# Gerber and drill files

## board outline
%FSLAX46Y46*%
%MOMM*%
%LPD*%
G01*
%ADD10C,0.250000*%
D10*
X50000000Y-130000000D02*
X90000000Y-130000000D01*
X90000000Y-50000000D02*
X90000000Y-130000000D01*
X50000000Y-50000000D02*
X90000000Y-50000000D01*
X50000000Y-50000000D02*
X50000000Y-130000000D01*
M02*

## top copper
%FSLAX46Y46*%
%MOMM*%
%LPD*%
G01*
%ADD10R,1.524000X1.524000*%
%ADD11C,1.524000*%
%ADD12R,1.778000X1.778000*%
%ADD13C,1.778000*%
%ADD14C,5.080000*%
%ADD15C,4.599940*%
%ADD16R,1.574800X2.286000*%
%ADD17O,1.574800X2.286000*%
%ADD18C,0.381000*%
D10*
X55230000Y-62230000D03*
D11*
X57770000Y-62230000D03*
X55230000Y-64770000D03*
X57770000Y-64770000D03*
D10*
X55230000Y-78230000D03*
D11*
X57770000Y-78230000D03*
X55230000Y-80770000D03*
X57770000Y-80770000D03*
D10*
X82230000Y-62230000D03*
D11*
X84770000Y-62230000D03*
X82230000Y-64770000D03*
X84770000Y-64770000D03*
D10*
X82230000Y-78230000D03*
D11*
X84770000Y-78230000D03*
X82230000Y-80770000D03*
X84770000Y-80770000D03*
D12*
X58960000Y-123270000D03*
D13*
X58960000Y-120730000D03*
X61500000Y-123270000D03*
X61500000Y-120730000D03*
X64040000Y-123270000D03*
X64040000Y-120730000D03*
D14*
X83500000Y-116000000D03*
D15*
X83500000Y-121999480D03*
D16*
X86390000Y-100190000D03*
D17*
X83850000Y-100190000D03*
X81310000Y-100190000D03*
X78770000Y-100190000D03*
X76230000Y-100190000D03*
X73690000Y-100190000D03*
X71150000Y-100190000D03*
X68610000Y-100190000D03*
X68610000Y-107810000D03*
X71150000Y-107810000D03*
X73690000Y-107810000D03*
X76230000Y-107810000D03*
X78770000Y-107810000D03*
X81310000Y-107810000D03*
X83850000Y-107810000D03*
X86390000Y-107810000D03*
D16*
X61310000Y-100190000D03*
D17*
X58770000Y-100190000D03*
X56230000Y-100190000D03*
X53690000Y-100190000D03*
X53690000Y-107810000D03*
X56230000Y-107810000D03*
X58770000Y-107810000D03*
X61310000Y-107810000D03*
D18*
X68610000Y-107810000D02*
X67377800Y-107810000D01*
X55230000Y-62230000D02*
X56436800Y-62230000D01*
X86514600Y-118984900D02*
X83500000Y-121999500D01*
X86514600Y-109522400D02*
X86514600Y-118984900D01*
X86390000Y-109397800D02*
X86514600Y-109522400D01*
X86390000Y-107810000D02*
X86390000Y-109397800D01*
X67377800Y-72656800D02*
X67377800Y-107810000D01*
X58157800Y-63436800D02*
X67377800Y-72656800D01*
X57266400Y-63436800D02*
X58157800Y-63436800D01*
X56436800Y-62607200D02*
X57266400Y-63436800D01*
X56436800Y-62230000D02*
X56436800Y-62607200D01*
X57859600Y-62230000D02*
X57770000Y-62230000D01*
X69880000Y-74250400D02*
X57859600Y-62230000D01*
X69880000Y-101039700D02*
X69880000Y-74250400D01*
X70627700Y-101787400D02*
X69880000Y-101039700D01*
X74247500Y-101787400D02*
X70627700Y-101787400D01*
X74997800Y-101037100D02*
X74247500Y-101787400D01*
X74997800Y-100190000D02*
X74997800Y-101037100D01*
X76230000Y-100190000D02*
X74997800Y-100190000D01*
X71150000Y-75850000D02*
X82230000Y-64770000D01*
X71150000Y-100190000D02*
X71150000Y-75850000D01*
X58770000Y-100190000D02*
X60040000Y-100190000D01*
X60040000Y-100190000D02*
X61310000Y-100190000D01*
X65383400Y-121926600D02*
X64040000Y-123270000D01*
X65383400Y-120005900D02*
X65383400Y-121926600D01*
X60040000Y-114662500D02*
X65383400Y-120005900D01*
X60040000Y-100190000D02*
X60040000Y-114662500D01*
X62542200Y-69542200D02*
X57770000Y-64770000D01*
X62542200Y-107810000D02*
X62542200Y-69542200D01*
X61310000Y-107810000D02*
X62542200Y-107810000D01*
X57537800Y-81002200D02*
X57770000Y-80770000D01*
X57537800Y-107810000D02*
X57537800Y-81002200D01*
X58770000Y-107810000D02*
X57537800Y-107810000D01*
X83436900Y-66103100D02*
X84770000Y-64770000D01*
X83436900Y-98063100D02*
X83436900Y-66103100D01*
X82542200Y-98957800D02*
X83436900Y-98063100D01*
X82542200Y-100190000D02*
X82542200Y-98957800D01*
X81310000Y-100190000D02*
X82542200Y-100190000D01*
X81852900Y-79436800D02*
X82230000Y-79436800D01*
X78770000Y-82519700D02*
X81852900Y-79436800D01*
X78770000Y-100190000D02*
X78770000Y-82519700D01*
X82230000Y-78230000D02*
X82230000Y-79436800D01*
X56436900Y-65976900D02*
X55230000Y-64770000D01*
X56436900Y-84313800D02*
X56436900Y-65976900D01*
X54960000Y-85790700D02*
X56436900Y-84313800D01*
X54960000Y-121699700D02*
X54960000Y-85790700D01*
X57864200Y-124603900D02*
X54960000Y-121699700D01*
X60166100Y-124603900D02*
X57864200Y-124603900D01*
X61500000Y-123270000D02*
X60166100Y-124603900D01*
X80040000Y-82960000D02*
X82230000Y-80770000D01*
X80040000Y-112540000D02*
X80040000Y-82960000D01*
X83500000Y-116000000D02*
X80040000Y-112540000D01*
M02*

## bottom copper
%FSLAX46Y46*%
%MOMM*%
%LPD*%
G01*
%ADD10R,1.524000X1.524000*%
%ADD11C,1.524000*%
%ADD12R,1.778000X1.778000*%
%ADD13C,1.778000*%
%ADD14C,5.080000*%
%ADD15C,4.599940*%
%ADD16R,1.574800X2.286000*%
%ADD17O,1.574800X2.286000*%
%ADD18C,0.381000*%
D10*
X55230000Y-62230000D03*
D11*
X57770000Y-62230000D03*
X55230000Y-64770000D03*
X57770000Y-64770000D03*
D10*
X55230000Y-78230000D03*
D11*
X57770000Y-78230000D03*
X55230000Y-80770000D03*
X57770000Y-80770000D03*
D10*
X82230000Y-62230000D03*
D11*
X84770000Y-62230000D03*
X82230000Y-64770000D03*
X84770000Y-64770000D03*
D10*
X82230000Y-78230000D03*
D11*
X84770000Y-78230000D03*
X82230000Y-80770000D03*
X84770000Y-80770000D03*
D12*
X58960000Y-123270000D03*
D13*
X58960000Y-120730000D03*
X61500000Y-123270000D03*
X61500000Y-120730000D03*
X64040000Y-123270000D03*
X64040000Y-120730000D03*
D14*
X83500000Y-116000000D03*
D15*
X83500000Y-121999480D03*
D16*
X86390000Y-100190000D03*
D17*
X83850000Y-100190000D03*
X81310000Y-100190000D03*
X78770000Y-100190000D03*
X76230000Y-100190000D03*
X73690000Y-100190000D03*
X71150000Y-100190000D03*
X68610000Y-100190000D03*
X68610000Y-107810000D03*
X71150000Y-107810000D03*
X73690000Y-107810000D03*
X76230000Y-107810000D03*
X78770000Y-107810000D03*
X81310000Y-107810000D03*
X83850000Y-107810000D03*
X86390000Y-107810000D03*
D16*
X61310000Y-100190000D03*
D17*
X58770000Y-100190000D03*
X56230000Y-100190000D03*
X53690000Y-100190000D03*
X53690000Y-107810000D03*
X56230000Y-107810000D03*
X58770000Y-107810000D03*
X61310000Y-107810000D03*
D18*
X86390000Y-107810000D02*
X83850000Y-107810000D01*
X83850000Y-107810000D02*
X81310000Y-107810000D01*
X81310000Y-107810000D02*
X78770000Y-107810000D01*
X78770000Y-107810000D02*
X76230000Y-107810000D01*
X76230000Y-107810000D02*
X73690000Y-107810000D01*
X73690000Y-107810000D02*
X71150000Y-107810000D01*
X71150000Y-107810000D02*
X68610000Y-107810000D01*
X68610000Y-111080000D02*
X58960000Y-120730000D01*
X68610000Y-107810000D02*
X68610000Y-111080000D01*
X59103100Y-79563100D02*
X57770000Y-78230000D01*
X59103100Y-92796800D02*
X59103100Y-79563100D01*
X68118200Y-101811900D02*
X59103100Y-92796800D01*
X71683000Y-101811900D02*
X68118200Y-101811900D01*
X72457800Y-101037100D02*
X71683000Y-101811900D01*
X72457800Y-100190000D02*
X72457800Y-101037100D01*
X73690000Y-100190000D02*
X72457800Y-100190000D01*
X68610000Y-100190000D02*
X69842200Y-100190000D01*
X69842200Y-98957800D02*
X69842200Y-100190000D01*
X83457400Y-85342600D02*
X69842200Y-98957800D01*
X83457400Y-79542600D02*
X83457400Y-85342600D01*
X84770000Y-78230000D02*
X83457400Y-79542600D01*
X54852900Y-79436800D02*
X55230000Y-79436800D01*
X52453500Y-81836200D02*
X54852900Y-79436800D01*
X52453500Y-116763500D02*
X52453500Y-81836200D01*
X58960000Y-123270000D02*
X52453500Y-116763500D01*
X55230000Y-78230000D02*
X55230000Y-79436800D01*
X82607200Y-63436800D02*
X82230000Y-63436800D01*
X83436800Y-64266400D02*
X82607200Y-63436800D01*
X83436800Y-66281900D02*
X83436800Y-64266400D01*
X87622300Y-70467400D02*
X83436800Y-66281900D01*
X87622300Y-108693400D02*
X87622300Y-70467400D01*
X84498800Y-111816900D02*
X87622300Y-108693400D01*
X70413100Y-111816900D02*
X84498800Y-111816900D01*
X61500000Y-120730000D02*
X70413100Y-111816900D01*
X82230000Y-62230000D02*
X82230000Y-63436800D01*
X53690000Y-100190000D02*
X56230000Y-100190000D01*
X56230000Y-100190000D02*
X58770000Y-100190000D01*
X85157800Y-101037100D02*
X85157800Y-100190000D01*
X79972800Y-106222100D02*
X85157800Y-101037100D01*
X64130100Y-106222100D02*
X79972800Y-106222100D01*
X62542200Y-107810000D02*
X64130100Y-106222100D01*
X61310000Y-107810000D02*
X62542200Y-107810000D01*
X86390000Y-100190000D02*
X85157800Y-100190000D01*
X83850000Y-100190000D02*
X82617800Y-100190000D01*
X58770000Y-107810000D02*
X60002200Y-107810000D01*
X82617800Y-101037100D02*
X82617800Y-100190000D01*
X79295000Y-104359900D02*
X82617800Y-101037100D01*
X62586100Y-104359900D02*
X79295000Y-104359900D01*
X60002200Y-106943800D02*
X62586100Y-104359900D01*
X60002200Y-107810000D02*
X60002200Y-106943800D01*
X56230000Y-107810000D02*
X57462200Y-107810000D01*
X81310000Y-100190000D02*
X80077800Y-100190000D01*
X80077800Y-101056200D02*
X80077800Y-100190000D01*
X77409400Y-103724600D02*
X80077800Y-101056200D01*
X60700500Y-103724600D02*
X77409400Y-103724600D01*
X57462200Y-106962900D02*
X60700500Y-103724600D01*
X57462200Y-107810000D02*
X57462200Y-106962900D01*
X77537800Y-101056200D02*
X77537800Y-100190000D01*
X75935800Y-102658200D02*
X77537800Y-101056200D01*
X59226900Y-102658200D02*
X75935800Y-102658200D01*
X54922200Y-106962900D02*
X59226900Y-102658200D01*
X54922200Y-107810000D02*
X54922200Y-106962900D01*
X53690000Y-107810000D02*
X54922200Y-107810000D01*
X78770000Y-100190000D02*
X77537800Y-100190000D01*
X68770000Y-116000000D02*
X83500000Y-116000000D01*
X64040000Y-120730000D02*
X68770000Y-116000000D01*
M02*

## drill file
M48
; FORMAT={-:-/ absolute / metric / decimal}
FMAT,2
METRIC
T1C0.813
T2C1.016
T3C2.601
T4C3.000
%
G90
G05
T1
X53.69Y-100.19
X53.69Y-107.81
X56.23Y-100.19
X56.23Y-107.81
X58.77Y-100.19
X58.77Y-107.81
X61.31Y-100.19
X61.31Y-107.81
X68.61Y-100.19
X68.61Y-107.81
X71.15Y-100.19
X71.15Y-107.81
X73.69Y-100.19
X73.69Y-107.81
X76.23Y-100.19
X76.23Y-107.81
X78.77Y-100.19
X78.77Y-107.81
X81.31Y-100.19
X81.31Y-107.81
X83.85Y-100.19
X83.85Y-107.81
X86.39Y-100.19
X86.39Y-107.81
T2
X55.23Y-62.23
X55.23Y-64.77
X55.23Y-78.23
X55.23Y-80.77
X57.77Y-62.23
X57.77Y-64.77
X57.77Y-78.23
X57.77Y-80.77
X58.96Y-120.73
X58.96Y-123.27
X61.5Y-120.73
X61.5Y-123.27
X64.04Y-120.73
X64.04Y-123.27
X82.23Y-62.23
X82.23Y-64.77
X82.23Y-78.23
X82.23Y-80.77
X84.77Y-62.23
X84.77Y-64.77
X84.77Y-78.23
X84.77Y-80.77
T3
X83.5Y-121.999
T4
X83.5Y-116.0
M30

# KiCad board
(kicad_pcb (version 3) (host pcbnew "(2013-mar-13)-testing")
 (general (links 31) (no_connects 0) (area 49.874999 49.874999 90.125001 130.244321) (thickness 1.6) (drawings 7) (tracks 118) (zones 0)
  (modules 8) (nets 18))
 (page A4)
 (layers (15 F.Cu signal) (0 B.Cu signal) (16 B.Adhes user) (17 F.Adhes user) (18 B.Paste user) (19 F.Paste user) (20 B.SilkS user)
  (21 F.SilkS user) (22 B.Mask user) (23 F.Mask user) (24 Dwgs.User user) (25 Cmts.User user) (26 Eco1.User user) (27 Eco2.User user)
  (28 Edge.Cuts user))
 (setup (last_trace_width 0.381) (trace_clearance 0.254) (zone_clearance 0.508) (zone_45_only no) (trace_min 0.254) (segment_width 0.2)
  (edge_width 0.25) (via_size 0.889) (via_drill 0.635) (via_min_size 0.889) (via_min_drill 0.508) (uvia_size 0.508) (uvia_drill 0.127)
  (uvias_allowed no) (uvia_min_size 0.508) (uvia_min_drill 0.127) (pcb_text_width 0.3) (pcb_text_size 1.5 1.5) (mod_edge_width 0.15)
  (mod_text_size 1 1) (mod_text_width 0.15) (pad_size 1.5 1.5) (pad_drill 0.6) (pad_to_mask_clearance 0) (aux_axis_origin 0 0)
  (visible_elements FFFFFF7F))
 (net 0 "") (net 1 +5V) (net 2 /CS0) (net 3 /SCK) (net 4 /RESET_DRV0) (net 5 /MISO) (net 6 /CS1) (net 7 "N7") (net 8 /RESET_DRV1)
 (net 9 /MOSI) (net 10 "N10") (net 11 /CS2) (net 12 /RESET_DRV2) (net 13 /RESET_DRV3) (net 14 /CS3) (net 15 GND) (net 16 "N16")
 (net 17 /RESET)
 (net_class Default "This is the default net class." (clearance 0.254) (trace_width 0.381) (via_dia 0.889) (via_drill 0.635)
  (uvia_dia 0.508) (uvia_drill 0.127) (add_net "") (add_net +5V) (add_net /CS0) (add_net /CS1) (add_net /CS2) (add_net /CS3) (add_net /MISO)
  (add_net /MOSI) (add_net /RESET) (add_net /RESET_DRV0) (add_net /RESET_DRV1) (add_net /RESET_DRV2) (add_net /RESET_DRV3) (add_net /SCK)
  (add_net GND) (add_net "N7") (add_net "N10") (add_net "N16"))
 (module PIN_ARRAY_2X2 (layer F.Cu) (at 56.5 63.5 270)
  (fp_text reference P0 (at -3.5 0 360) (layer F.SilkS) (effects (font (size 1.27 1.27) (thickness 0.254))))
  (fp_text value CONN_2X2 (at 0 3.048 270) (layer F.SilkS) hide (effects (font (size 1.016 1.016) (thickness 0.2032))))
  (pad 1 thru_hole rect (at -1.27 1.27 270) (size 1.524 1.524) (drill 1.016) (layers *.Cu *.Mask F.SilkS) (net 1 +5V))
  (pad 2 thru_hole circle (at -1.27 -1.27 270) (size 1.524 1.524) (drill 1.016) (layers *.Cu *.Mask F.SilkS) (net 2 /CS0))
  (pad 3 thru_hole circle (at 1.27 1.27 270) (size 1.524 1.524) (drill 1.016) (layers *.Cu *.Mask F.SilkS) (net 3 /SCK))
  (pad 4 thru_hole circle (at 1.27 -1.27 270) (size 1.524 1.524) (drill 1.016) (layers *.Cu *.Mask F.SilkS) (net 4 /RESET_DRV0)))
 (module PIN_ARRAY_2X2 (layer F.Cu) (at 56.5 79.5 270)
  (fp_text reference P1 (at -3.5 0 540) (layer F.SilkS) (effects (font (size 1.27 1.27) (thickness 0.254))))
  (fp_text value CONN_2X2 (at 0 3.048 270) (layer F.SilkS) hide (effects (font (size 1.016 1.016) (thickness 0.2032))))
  (pad 1 thru_hole rect (at -1.27 1.27 270) (size 1.524 1.524) (drill 1.016) (layers *.Cu *.Mask F.SilkS) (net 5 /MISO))
  (pad 2 thru_hole circle (at -1.27 -1.27 270) (size 1.524 1.524) (drill 1.016) (layers *.Cu *.Mask F.SilkS) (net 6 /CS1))
  (pad 3 thru_hole circle (at 1.27 1.27 270) (size 1.524 1.524) (drill 1.016) (layers *.Cu *.Mask F.SilkS) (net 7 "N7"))
  (pad 4 thru_hole circle (at 1.27 -1.27 270) (size 1.524 1.524) (drill 1.016) (layers *.Cu *.Mask F.SilkS) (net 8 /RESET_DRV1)))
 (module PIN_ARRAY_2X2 (layer F.Cu) (at 83.5 63.5 270)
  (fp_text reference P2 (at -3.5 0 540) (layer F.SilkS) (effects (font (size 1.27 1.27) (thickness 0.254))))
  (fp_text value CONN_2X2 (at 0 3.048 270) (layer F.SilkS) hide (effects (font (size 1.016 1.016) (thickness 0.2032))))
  (pad 1 thru_hole rect (at -1.27 1.27 270) (size 1.524 1.524) (drill 1.016) (layers *.Cu *.Mask F.SilkS) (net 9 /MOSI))
  (pad 2 thru_hole circle (at -1.27 -1.27 270) (size 1.524 1.524) (drill 1.016) (layers *.Cu *.Mask F.SilkS) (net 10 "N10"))
  (pad 3 thru_hole circle (at 1.27 1.27 270) (size 1.524 1.524) (drill 1.016) (layers *.Cu *.Mask F.SilkS) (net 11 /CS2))
  (pad 4 thru_hole circle (at 1.27 -1.27 270) (size 1.524 1.524) (drill 1.016) (layers *.Cu *.Mask F.SilkS) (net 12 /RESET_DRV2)))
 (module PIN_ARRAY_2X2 (layer F.Cu) (at 83.5 79.5 270)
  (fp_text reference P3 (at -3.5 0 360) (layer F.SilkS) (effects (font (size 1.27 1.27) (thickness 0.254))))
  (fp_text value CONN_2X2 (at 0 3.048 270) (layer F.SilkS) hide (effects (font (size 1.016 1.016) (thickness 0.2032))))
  (pad 1 thru_hole rect (at -1.27 1.27 270) (size 1.524 1.524) (drill 1.016) (layers *.Cu *.Mask F.SilkS) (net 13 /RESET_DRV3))
  (pad 2 thru_hole circle (at -1.27 -1.27 270) (size 1.524 1.524) (drill 1.016) (layers *.Cu *.Mask F.SilkS) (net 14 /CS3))
  (pad 3 thru_hole circle (at 1.27 1.27 270) (size 1.524 1.524) (drill 1.016) (layers *.Cu *.Mask F.SilkS) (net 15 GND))
  (pad 4 thru_hole circle (at 1.27 -1.27 270) (size 1.524 1.524) (drill 1.016) (layers *.Cu *.Mask F.SilkS) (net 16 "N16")))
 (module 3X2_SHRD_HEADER (layer F.Cu) (at 61.5 122)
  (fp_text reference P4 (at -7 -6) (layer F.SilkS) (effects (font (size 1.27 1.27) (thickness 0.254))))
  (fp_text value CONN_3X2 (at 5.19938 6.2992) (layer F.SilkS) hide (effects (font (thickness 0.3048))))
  (pad 1 thru_hole rect (at -2.54 1.27) (size 1.778 1.778) (drill 1.016) (layers *.Cu *.Mask F.SilkS) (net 5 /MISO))
  (pad 2 thru_hole circle (at -2.54 -1.27) (size 1.778 1.778) (drill 1.016) (layers *.Cu *.Mask F.SilkS) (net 1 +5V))
  (pad 3 thru_hole circle (at 0 1.27) (size 1.778 1.778) (drill 1.016) (layers *.Cu *.Mask F.SilkS) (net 3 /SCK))
  (pad 4 thru_hole circle (at 0 -1.27) (size 1.778 1.778) (drill 1.016) (layers *.Cu *.Mask F.SilkS) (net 9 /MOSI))
  (pad 5 thru_hole circle (at 2.54 1.27) (size 1.778 1.778) (drill 1.016) (layers *.Cu *.Mask F.SilkS) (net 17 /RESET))
  (pad 6 thru_hole circle (at 2.54 -1.27) (size 1.778 1.778) (drill 1.016) (layers *.Cu *.Mask F.SilkS) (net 15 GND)))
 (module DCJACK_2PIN (layer F.Cu) (at 83.5 116 270)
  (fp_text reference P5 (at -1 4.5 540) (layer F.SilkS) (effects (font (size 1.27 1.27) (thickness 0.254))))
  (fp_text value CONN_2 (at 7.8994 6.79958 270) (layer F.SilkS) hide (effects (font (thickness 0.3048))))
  (pad 1 thru_hole circle (at 0 0 270) (size 5.08 5.08) (drill 2.99974) (layers *.Cu *.Mask F.SilkS) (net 15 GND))
  (pad 2 thru_hole circle (at 5.99948 0 270) (size 4.59994 4.59994) (drill 2.60096) (layers *.Cu *.Mask F.SilkS) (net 1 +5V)))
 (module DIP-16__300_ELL (layer F.Cu) (at 77.5 104 180)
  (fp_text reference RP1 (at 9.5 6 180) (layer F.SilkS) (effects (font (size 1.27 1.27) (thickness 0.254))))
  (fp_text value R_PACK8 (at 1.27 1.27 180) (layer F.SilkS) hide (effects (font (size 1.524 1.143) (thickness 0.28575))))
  (pad 1 thru_hole rect (at -8.89 3.81 180) (size 1.5748 2.286) (drill 0.8128) (layers *.Cu *.Mask F.SilkS) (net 4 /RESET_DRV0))
  (pad 2 thru_hole oval (at -6.35 3.81 180) (size 1.5748 2.286) (drill 0.8128) (layers *.Cu *.Mask F.SilkS) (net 8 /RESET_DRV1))
  (pad 3 thru_hole oval (at -3.81 3.81 180) (size 1.5748 2.286) (drill 0.8128) (layers *.Cu *.Mask F.SilkS) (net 12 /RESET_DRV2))
  (pad 4 thru_hole oval (at -1.27 3.81 180) (size 1.5748 2.286) (drill 0.8128) (layers *.Cu *.Mask F.SilkS) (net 13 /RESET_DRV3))
  (pad 5 thru_hole oval (at 1.27 3.81 180) (size 1.5748 2.286) (drill 0.8128) (layers *.Cu *.Mask F.SilkS) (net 2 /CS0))
  (pad 6 thru_hole oval (at 3.81 3.81 180) (size 1.5748 2.286) (drill 0.8128) (layers *.Cu *.Mask F.SilkS) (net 6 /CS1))
  (pad 7 thru_hole oval (at 6.35 3.81 180) (size 1.5748 2.286) (drill 0.8128) (layers *.Cu *.Mask F.SilkS) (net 11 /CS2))
  (pad 8 thru_hole oval (at 8.89 3.81 180) (size 1.5748 2.286) (drill 0.8128) (layers *.Cu *.Mask F.SilkS) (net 14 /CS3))
  (pad 9 thru_hole oval (at 8.89 -3.81 180) (size 1.5748 2.286) (drill 0.8128) (layers *.Cu *.Mask F.SilkS) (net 1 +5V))
  (pad 10 thru_hole oval (at 6.35 -3.81 180) (size 1.5748 2.286) (drill 0.8128) (layers *.Cu *.Mask F.SilkS) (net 1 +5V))
  (pad 11 thru_hole oval (at 3.81 -3.81 180) (size 1.5748 2.286) (drill 0.8128) (layers *.Cu *.Mask F.SilkS) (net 1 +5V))
  (pad 12 thru_hole oval (at 1.27 -3.81 180) (size 1.5748 2.286) (drill 0.8128) (layers *.Cu *.Mask F.SilkS) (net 1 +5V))
  (pad 13 thru_hole oval (at -1.27 -3.81 180) (size 1.5748 2.286) (drill 0.8128) (layers *.Cu *.Mask F.SilkS) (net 1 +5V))
  (pad 14 thru_hole oval (at -3.81 -3.81 180) (size 1.5748 2.286) (drill 0.8128) (layers *.Cu *.Mask F.SilkS) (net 1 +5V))
  (pad 15 thru_hole oval (at -6.35 -3.81 180) (size 1.5748 2.286) (drill 0.8128) (layers *.Cu *.Mask F.SilkS) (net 1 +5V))
  (pad 16 thru_hole oval (at -8.89 -3.81 180) (size 1.5748 2.286) (drill 0.8128) (layers *.Cu *.Mask F.SilkS) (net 1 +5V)))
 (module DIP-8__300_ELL (layer F.Cu) (at 57.5 104 180)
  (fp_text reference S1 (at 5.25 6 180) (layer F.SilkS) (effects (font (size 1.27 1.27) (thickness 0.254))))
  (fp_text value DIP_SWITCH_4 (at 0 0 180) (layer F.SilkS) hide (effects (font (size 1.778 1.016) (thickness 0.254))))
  (pad 1 thru_hole rect (at -3.81 3.81 180) (size 1.5748 2.286) (drill 0.8128) (layers *.Cu *.Mask F.SilkS) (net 17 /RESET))
  (pad 2 thru_hole oval (at -1.27 3.81 180) (size 1.5748 2.286) (drill 0.8128) (layers *.Cu *.Mask F.SilkS) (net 17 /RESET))
  (pad 3 thru_hole oval (at 1.27 3.81 180) (size 1.5748 2.286) (drill 0.8128) (layers *.Cu *.Mask F.SilkS) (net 17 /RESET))
  (pad 4 thru_hole oval (at 3.81 3.81 180) (size 1.5748 2.286) (drill 0.8128) (layers *.Cu *.Mask F.SilkS) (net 17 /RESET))
  (pad 5 thru_hole oval (at 3.81 -3.81 180) (size 1.5748 2.286) (drill 0.8128) (layers *.Cu *.Mask F.SilkS) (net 13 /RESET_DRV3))
  (pad 6 thru_hole oval (at 1.27 -3.81 180) (size 1.5748 2.286) (drill 0.8128) (layers *.Cu *.Mask F.SilkS) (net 12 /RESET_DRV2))
  (pad 7 thru_hole oval (at -1.27 -3.81 180) (size 1.5748 2.286) (drill 0.8128) (layers *.Cu *.Mask F.SilkS) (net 8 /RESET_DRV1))
  (pad 8 thru_hole oval (at -3.81 -3.81 180) (size 1.5748 2.286) (drill 0.8128) (layers *.Cu *.Mask F.SilkS) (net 4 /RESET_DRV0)))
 (gr_line (start 50 130) (end 90 130) (angle 90) (layer Edge.Cuts) (width 0.25))
 (gr_line (start 90 50) (end 90 130) (angle 90) (layer Edge.Cuts) (width 0.25))
 (gr_line (start 50 50) (end 90 50) (angle 90) (layer Edge.Cuts) (width 0.25))
 (gr_line (start 50 50) (end 50 130) (angle 90) (layer Edge.Cuts) (width 0.25))
 (segment (start 86.39 107.81) (end 83.85 107.81) (width 0.381) (layer B.Cu) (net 1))
 (segment (start 83.85 107.81) (end 81.31 107.81) (width 0.381) (layer B.Cu) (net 1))
 (segment (start 81.31 107.81) (end 78.77 107.81) (width 0.381) (layer B.Cu) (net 1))
 (segment (start 78.77 107.81) (end 76.23 107.81) (width 0.381) (layer B.Cu) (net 1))
 (segment (start 76.23 107.81) (end 73.69 107.81) (width 0.381) (layer B.Cu) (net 1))
 (segment (start 73.69 107.81) (end 71.15 107.81) (width 0.381) (layer B.Cu) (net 1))
 (segment (start 71.15 107.81) (end 68.61 107.81) (width 0.381) (layer B.Cu) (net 1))
 (segment (start 68.61 111.08) (end 58.96 120.73) (width 0.381) (layer B.Cu) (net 1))
 (segment (start 68.61 107.81) (end 68.61 111.08) (width 0.381) (layer B.Cu) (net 1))
 (segment (start 68.61 107.81) (end 67.3778 107.81) (width 0.381) (layer F.Cu) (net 1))
 (segment (start 55.23 62.23) (end 56.4368 62.23) (width 0.381) (layer F.Cu) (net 1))
 (segment (start 86.5146 118.9849) (end 83.5 121.9995) (width 0.381) (layer F.Cu) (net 1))
 (segment (start 86.5146 109.5224) (end 86.5146 118.9849) (width 0.381) (layer F.Cu) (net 1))
 (segment (start 86.39 109.3978) (end 86.5146 109.5224) (width 0.381) (layer F.Cu) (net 1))
 (segment (start 86.39 107.81) (end 86.39 109.3978) (width 0.381) (layer F.Cu) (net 1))
 (segment (start 67.3778 72.6568) (end 67.3778 107.81) (width 0.381) (layer F.Cu) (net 1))
 (segment (start 58.1578 63.4368) (end 67.3778 72.6568) (width 0.381) (layer F.Cu) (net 1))
 (segment (start 57.2664 63.4368) (end 58.1578 63.4368) (width 0.381) (layer F.Cu) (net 1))
 (segment (start 56.4368 62.6072) (end 57.2664 63.4368) (width 0.381) (layer F.Cu) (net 1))
 (segment (start 56.4368 62.23) (end 56.4368 62.6072) (width 0.381) (layer F.Cu) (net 1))
 (segment (start 57.8596 62.23) (end 57.77 62.23) (width 0.381) (layer F.Cu) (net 2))
 (segment (start 69.88 74.2504) (end 57.8596 62.23) (width 0.381) (layer F.Cu) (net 2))
 (segment (start 69.88 101.0397) (end 69.88 74.2504) (width 0.381) (layer F.Cu) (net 2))
 (segment (start 70.6277 101.7874) (end 69.88 101.0397) (width 0.381) (layer F.Cu) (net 2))
 (segment (start 74.2475 101.7874) (end 70.6277 101.7874) (width 0.381) (layer F.Cu) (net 2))
 (segment (start 74.9978 101.0371) (end 74.2475 101.7874) (width 0.381) (layer F.Cu) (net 2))
 (segment (start 74.9978 100.19) (end 74.9978 101.0371) (width 0.381) (layer F.Cu) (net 2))
 (segment (start 76.23 100.19) (end 74.9978 100.19) (width 0.381) (layer F.Cu) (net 2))
 (segment (start 59.1031 79.5631) (end 57.77 78.23) (width 0.381) (layer B.Cu) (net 6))
 (segment (start 59.1031 92.7968) (end 59.1031 79.5631) (width 0.381) (layer B.Cu) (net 6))
 (segment (start 68.1182 101.8119) (end 59.1031 92.7968) (width 0.381) (layer B.Cu) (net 6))
 (segment (start 71.683 101.8119) (end 68.1182 101.8119) (width 0.381) (layer B.Cu) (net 6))
 (segment (start 72.4578 101.0371) (end 71.683 101.8119) (width 0.381) (layer B.Cu) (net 6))
 (segment (start 72.4578 100.19) (end 72.4578 101.0371) (width 0.381) (layer B.Cu) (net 6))
 (segment (start 73.69 100.19) (end 72.4578 100.19) (width 0.381) (layer B.Cu) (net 6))
 (segment (start 71.15 75.85) (end 82.23 64.77) (width 0.381) (layer F.Cu) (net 11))
 (segment (start 71.15 100.19) (end 71.15 75.85) (width 0.381) (layer F.Cu) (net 11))
 (segment (start 68.61 100.19) (end 69.8422 100.19) (width 0.381) (layer B.Cu) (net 14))
 (segment (start 69.8422 98.9578) (end 69.8422 100.19) (width 0.381) (layer B.Cu) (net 14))
 (segment (start 83.4574 85.3426) (end 69.8422 98.9578) (width 0.381) (layer B.Cu) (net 14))
 (segment (start 83.4574 79.5426) (end 83.4574 85.3426) (width 0.381) (layer B.Cu) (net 14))
 (segment (start 84.77 78.23) (end 83.4574 79.5426) (width 0.381) (layer B.Cu) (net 14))
 (segment (start 54.8529 79.4368) (end 55.23 79.4368) (width 0.381) (layer B.Cu) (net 5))
 (segment (start 52.4535 81.8362) (end 54.8529 79.4368) (width 0.381) (layer B.Cu) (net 5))
 (segment (start 52.4535 116.7635) (end 52.4535 81.8362) (width 0.381) (layer B.Cu) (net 5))
 (segment (start 58.96 123.27) (end 52.4535 116.7635) (width 0.381) (layer B.Cu) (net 5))
 (segment (start 55.23 78.23) (end 55.23 79.4368) (width 0.381) (layer B.Cu) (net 5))
 (segment (start 82.6072 63.4368) (end 82.23 63.4368) (width 0.381) (layer B.Cu) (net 9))
 (segment (start 83.4368 64.2664) (end 82.6072 63.4368) (width 0.381) (layer B.Cu) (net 9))
 (segment (start 83.4368 66.2819) (end 83.4368 64.2664) (width 0.381) (layer B.Cu) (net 9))
 (segment (start 87.6223 70.4674) (end 83.4368 66.2819) (width 0.381) (layer B.Cu) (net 9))
 (segment (start 87.6223 108.6934) (end 87.6223 70.4674) (width 0.381) (layer B.Cu) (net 9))
 (segment (start 84.4988 111.8169) (end 87.6223 108.6934) (width 0.381) (layer B.Cu) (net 9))
 (segment (start 70.4131 111.8169) (end 84.4988 111.8169) (width 0.381) (layer B.Cu) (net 9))
 (segment (start 61.5 120.73) (end 70.4131 111.8169) (width 0.381) (layer B.Cu) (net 9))
 (segment (start 82.23 62.23) (end 82.23 63.4368) (width 0.381) (layer B.Cu) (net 9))
 (segment (start 53.69 100.19) (end 56.23 100.19) (width 0.381) (layer B.Cu) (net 17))
 (segment (start 56.23 100.19) (end 58.77 100.19) (width 0.381) (layer B.Cu) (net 17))
 (segment (start 58.77 100.19) (end 60.04 100.19) (width 0.381) (layer F.Cu) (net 17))
 (segment (start 60.04 100.19) (end 61.31 100.19) (width 0.381) (layer F.Cu) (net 17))
 (segment (start 65.3834 121.9266) (end 64.04 123.27) (width 0.381) (layer F.Cu) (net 17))
 (segment (start 65.3834 120.0059) (end 65.3834 121.9266) (width 0.381) (layer F.Cu) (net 17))
 (segment (start 60.04 114.6625) (end 65.3834 120.0059) (width 0.381) (layer F.Cu) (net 17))
 (segment (start 60.04 100.19) (end 60.04 114.6625) (width 0.381) (layer F.Cu) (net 17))
 (segment (start 62.5422 69.5422) (end 57.77 64.77) (width 0.381) (layer F.Cu) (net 4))
 (segment (start 62.5422 107.81) (end 62.5422 69.5422) (width 0.381) (layer F.Cu) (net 4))
 (segment (start 61.31 107.81) (end 62.5422 107.81) (width 0.381) (layer F.Cu) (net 4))
 (segment (start 85.1578 101.0371) (end 85.1578 100.19) (width 0.381) (layer B.Cu) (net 4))
 (segment (start 79.9728 106.2221) (end 85.1578 101.0371) (width 0.381) (layer B.Cu) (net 4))
 (segment (start 64.1301 106.2221) (end 79.9728 106.2221) (width 0.381) (layer B.Cu) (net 4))
 (segment (start 62.5422 107.81) (end 64.1301 106.2221) (width 0.381) (layer B.Cu) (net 4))
 (segment (start 61.31 107.81) (end 62.5422 107.81) (width 0.381) (layer B.Cu) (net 4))
 (segment (start 86.39 100.19) (end 85.1578 100.19) (width 0.381) (layer B.Cu) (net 4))
 (segment (start 57.5378 81.0022) (end 57.77 80.77) (width 0.381) (layer F.Cu) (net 8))
 (segment (start 57.5378 107.81) (end 57.5378 81.0022) (width 0.381) (layer F.Cu) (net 8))
 (segment (start 58.77 107.81) (end 57.5378 107.81) (width 0.381) (layer F.Cu) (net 8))
 (segment (start 83.85 100.19) (end 82.6178 100.19) (width 0.381) (layer B.Cu) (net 8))
 (segment (start 58.77 107.81) (end 60.0022 107.81) (width 0.381) (layer B.Cu) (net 8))
 (segment (start 82.6178 101.0371) (end 82.6178 100.19) (width 0.381) (layer B.Cu) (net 8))
 (segment (start 79.295 104.3599) (end 82.6178 101.0371) (width 0.381) (layer B.Cu) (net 8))
 (segment (start 62.5861 104.3599) (end 79.295 104.3599) (width 0.381) (layer B.Cu) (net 8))
 (segment (start 60.0022 106.9438) (end 62.5861 104.3599) (width 0.381) (layer B.Cu) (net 8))
 (segment (start 60.0022 107.81) (end 60.0022 106.9438) (width 0.381) (layer B.Cu) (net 8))
 (segment (start 56.23 107.81) (end 57.4622 107.81) (width 0.381) (layer B.Cu) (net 12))
 (segment (start 81.31 100.19) (end 80.0778 100.19) (width 0.381) (layer B.Cu) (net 12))
 (segment (start 80.0778 101.0562) (end 80.0778 100.19) (width 0.381) (layer B.Cu) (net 12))
 (segment (start 77.4094 103.7246) (end 80.0778 101.0562) (width 0.381) (layer B.Cu) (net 12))
 (segment (start 60.7005 103.7246) (end 77.4094 103.7246) (width 0.381) (layer B.Cu) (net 12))
 (segment (start 57.4622 106.9629) (end 60.7005 103.7246) (width 0.381) (layer B.Cu) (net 12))
 (segment (start 57.4622 107.81) (end 57.4622 106.9629) (width 0.381) (layer B.Cu) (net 12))
 (segment (start 83.4369 66.1031) (end 84.77 64.77) (width 0.381) (layer F.Cu) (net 12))
 (segment (start 83.4369 98.0631) (end 83.4369 66.1031) (width 0.381) (layer F.Cu) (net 12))
 (segment (start 82.5422 98.9578) (end 83.4369 98.0631) (width 0.381) (layer F.Cu) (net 12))
 (segment (start 82.5422 100.19) (end 82.5422 98.9578) (width 0.381) (layer F.Cu) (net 12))
 (segment (start 81.31 100.19) (end 82.5422 100.19) (width 0.381) (layer F.Cu) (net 12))
 (segment (start 81.8529 79.4368) (end 82.23 79.4368) (width 0.381) (layer F.Cu) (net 13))
 (segment (start 78.77 82.5197) (end 81.8529 79.4368) (width 0.381) (layer F.Cu) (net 13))
 (segment (start 78.77 100.19) (end 78.77 82.5197) (width 0.381) (layer F.Cu) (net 13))
 (segment (start 82.23 78.23) (end 82.23 79.4368) (width 0.381) (layer F.Cu) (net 13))
 (segment (start 77.5378 101.0562) (end 77.5378 100.19) (width 0.381) (layer B.Cu) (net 13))
 (segment (start 75.9358 102.6582) (end 77.5378 101.0562) (width 0.381) (layer B.Cu) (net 13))
 (segment (start 59.2269 102.6582) (end 75.9358 102.6582) (width 0.381) (layer B.Cu) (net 13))
 (segment (start 54.9222 106.9629) (end 59.2269 102.6582) (width 0.381) (layer B.Cu) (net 13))
 (segment (start 54.9222 107.81) (end 54.9222 106.9629) (width 0.381) (layer B.Cu) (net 13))
 (segment (start 53.69 107.81) (end 54.9222 107.81) (width 0.381) (layer B.Cu) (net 13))
 (segment (start 78.77 100.19) (end 77.5378 100.19) (width 0.381) (layer B.Cu) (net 13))
 (segment (start 56.4369 65.9769) (end 55.23 64.77) (width 0.381) (layer F.Cu) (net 3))
 (segment (start 56.4369 84.3138) (end 56.4369 65.9769) (width 0.381) (layer F.Cu) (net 3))
 (segment (start 54.96 85.7907) (end 56.4369 84.3138) (width 0.381) (layer F.Cu) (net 3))
 (segment (start 54.96 121.6997) (end 54.96 85.7907) (width 0.381) (layer F.Cu) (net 3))
 (segment (start 57.8642 124.6039) (end 54.96 121.6997) (width 0.381) (layer F.Cu) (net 3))
 (segment (start 60.1661 124.6039) (end 57.8642 124.6039) (width 0.381) (layer F.Cu) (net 3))
 (segment (start 61.5 123.27) (end 60.1661 124.6039) (width 0.381) (layer F.Cu) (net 3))
 (segment (start 80.04 82.96) (end 82.23 80.77) (width 0.381) (layer F.Cu) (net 15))
 (segment (start 80.04 112.54) (end 80.04 82.96) (width 0.381) (layer F.Cu) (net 15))
 (segment (start 83.5 116) (end 80.04 112.54) (width 0.381) (layer F.Cu) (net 15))
 (segment (start 68.77 116) (end 83.5 116) (width 0.381) (layer B.Cu) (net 15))
 (segment (start 64.04 120.73) (end 68.77 116) (width 0.381) (layer B.Cu) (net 15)))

